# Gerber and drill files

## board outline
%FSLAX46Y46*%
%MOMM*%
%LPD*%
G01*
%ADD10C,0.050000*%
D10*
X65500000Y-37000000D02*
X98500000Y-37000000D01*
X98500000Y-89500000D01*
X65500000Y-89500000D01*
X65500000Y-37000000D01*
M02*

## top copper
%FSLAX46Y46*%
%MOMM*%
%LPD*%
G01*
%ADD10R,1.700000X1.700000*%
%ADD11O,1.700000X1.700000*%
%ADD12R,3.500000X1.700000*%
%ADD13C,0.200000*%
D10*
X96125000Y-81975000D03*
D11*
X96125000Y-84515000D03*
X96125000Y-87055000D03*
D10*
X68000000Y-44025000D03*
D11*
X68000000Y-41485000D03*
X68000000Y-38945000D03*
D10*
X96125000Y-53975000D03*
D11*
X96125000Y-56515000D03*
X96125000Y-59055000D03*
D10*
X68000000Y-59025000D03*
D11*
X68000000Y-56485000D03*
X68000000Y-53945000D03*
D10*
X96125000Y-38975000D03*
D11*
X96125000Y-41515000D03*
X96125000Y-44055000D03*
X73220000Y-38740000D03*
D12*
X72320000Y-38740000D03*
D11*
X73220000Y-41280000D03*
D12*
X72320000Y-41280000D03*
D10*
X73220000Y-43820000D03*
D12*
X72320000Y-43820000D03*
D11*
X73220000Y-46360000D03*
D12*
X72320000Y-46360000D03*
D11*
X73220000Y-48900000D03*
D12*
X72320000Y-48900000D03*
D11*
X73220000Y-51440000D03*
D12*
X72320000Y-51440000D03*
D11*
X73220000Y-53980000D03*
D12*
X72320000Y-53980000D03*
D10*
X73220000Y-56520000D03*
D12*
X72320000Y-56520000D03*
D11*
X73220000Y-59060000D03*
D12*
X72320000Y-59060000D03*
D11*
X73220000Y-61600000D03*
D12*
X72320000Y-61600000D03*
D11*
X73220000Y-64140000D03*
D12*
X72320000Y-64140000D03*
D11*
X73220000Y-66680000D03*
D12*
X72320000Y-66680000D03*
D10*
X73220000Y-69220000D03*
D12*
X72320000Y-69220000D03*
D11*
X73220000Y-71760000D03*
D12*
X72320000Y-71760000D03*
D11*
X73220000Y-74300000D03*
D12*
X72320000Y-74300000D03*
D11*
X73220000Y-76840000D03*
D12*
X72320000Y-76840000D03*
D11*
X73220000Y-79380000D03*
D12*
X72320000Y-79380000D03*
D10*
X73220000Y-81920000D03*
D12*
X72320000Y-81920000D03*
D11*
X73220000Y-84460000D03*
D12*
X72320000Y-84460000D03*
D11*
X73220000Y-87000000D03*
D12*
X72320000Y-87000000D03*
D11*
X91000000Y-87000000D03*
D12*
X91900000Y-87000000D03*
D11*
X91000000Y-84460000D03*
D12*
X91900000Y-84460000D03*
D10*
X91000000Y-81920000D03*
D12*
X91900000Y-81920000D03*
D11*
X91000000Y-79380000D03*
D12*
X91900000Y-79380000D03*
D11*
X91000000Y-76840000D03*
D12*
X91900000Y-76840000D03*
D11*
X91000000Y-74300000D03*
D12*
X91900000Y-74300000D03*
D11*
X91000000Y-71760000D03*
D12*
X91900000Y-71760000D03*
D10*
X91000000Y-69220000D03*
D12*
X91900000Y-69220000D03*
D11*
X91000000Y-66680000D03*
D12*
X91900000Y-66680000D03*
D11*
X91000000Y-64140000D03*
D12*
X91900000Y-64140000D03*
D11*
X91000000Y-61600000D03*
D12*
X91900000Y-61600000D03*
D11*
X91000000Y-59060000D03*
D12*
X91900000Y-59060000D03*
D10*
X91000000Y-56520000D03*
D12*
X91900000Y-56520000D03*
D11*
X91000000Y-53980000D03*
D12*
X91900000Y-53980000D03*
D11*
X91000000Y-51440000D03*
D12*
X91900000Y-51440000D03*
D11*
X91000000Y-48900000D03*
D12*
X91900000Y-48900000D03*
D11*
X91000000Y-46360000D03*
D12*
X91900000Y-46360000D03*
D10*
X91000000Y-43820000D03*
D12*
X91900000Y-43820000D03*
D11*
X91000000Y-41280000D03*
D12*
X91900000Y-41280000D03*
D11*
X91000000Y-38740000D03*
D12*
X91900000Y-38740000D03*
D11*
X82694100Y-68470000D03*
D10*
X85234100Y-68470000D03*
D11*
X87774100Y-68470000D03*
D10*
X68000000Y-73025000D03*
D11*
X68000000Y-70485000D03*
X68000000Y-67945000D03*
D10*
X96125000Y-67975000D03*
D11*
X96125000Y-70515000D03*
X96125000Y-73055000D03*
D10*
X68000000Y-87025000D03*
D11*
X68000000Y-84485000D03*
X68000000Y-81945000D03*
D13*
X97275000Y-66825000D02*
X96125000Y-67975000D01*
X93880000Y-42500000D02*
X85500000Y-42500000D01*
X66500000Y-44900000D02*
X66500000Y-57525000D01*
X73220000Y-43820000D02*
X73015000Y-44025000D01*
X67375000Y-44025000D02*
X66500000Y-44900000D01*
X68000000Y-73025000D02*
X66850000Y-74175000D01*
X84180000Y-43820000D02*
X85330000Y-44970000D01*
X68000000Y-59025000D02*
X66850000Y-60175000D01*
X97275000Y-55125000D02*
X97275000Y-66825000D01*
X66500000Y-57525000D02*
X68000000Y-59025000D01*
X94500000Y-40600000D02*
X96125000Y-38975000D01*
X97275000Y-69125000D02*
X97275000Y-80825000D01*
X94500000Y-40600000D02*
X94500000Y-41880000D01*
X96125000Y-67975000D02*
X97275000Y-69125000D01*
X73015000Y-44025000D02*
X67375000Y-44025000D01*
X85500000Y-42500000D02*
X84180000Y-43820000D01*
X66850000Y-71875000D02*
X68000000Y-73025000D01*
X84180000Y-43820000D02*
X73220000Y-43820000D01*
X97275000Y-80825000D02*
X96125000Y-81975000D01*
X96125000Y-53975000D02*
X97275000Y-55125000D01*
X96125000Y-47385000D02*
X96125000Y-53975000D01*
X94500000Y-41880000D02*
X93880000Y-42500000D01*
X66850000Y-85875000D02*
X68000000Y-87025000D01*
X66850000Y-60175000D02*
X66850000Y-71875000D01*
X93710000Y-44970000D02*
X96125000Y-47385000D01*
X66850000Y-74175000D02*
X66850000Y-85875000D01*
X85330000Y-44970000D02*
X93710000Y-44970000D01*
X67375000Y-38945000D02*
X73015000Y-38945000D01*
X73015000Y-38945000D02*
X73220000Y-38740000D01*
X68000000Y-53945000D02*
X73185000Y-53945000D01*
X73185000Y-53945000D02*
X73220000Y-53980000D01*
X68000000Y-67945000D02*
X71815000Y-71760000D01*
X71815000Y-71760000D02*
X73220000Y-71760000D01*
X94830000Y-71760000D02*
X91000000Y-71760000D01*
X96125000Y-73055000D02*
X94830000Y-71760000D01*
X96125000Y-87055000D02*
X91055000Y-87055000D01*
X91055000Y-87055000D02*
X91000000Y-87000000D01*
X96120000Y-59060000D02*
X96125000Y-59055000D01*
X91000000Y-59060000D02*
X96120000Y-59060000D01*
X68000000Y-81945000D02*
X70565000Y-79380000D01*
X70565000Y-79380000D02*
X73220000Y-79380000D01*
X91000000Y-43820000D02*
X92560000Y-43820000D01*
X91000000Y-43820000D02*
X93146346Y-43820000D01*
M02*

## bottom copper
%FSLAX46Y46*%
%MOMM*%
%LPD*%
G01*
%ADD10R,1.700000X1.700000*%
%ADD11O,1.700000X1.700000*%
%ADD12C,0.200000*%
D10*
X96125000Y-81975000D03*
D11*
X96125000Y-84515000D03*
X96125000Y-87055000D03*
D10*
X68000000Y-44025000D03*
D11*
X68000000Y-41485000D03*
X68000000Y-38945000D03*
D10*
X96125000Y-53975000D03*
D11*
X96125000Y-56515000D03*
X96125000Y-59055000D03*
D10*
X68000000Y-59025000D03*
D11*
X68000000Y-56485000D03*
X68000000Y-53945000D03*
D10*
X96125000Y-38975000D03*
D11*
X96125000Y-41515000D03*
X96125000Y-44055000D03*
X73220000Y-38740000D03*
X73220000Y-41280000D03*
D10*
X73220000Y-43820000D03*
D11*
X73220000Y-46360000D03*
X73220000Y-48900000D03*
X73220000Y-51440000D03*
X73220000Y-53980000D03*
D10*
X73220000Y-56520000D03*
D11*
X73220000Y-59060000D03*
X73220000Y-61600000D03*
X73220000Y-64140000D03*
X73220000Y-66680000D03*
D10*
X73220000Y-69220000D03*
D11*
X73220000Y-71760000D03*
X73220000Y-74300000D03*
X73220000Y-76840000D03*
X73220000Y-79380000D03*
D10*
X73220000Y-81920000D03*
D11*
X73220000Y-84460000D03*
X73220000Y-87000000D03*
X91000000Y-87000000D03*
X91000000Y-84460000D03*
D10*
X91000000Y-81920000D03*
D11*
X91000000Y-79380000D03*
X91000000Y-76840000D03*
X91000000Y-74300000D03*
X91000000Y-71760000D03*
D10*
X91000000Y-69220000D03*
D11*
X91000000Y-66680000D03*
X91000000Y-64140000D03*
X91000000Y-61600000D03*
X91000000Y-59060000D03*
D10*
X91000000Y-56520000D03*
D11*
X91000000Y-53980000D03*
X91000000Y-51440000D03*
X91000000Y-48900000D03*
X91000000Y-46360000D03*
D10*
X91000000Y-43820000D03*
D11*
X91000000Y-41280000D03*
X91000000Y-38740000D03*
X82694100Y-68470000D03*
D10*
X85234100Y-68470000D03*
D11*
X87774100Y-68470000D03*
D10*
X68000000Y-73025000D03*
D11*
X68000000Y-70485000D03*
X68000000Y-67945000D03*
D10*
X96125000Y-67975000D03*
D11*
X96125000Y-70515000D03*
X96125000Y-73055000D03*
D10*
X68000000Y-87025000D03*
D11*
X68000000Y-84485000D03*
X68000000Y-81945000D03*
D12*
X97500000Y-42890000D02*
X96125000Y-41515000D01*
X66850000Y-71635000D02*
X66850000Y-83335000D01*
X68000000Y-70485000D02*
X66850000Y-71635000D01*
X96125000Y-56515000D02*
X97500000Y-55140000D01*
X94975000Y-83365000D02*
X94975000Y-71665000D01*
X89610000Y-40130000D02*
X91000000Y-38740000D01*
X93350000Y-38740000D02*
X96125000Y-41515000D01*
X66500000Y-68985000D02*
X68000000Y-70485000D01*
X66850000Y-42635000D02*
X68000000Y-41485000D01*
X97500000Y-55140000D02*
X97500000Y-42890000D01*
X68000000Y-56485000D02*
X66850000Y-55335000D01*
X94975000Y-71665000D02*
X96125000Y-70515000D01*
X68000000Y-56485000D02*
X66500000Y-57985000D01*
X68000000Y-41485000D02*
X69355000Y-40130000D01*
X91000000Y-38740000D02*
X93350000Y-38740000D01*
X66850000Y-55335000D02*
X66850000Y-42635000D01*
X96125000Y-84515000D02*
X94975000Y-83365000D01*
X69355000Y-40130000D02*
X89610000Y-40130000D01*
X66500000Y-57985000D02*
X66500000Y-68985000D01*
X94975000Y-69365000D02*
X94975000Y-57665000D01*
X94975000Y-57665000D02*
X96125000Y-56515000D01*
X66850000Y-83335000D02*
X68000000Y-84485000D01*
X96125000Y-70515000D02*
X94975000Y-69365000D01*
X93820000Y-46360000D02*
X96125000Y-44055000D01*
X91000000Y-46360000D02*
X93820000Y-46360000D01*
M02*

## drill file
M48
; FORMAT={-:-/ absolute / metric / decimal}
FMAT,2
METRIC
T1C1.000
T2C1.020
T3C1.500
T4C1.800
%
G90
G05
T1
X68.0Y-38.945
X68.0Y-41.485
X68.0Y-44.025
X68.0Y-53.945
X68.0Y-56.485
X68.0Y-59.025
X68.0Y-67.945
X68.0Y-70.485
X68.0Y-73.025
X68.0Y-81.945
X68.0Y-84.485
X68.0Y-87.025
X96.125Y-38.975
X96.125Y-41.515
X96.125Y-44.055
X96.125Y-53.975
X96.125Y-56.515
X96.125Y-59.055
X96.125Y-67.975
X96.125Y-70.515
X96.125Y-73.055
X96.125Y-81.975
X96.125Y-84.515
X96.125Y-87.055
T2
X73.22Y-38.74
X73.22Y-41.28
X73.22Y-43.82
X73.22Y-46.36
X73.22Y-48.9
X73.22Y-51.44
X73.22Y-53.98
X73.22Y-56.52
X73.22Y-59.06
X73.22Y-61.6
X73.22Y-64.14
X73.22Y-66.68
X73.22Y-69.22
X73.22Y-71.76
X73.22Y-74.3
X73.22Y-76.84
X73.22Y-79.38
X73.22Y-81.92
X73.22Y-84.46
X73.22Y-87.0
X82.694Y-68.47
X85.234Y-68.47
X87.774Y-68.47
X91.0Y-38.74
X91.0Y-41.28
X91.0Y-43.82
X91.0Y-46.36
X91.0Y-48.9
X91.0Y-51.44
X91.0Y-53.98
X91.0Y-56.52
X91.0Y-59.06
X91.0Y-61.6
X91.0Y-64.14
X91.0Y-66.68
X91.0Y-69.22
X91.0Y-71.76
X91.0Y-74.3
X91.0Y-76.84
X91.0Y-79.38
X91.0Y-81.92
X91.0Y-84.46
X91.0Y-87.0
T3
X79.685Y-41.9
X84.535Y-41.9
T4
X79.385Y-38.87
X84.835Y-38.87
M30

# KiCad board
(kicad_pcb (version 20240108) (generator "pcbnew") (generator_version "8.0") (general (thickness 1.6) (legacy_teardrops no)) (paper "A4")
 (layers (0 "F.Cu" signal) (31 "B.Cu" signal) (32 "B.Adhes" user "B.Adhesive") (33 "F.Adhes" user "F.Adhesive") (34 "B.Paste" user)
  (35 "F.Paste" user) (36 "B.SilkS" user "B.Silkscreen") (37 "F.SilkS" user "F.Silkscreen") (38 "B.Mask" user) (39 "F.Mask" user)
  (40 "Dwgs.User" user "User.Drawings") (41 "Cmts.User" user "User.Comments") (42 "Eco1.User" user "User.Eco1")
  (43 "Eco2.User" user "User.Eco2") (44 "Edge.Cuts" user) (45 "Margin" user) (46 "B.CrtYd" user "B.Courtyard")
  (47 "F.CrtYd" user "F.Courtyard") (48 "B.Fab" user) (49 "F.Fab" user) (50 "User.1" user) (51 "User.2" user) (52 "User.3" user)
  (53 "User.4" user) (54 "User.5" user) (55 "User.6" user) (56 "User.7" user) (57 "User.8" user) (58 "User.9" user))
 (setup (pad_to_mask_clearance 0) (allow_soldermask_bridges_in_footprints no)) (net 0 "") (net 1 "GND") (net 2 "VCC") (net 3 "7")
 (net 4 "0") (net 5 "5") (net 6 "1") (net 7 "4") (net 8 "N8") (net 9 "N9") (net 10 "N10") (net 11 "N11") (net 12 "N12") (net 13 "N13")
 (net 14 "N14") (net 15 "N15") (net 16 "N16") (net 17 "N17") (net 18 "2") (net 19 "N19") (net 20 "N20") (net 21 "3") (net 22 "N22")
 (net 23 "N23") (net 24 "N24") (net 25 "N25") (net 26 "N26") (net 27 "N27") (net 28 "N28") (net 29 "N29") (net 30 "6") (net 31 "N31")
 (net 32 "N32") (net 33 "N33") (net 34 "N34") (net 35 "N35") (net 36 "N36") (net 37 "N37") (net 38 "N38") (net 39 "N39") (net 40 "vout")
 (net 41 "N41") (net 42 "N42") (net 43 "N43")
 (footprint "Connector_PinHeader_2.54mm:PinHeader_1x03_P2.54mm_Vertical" (layer "F.Cu") (at 96.125 81.975)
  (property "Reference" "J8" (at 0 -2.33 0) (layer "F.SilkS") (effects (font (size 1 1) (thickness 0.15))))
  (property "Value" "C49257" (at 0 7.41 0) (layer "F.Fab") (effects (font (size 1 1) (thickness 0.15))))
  (pad "1" thru_hole rect (at 0 0) (size 1.7 1.7) (drill 1) (layers "*.Cu" "*.Mask") (remove_unused_layers no) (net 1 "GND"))
  (pad "2" thru_hole oval (at 0 2.54) (size 1.7 1.7) (drill 1) (layers "*.Cu" "*.Mask") (remove_unused_layers no) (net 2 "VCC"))
  (pad "3" thru_hole oval (at 0 5.08) (size 1.7 1.7) (drill 1) (layers "*.Cu" "*.Mask") (remove_unused_layers no) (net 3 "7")))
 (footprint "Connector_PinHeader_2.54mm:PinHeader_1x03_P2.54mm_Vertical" (layer "F.Cu") (at 68 44.025 180)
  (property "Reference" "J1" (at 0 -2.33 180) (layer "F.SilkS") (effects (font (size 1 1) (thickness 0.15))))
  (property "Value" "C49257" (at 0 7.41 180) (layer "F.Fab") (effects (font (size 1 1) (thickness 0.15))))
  (pad "1" thru_hole rect (at 0 0 180) (size 1.7 1.7) (drill 1) (layers "*.Cu" "*.Mask") (remove_unused_layers no) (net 1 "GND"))
  (pad "2" thru_hole oval (at 0 2.54 180) (size 1.7 1.7) (drill 1) (layers "*.Cu" "*.Mask") (remove_unused_layers no) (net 2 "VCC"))
  (pad "3" thru_hole oval (at 0 5.08 180) (size 1.7 1.7) (drill 1) (layers "*.Cu" "*.Mask") (remove_unused_layers no) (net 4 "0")))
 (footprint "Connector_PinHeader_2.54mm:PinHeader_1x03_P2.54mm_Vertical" (layer "F.Cu") (at 96.125 53.975)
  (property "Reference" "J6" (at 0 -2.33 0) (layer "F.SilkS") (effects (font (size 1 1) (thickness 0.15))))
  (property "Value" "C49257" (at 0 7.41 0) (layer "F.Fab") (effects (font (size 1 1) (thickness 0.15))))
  (pad "1" thru_hole rect (at 0 0) (size 1.7 1.7) (drill 1) (layers "*.Cu" "*.Mask") (remove_unused_layers no) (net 1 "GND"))
  (pad "2" thru_hole oval (at 0 2.54) (size 1.7 1.7) (drill 1) (layers "*.Cu" "*.Mask") (remove_unused_layers no) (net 2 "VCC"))
  (pad "3" thru_hole oval (at 0 5.08) (size 1.7 1.7) (drill 1) (layers "*.Cu" "*.Mask") (remove_unused_layers no) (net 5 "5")))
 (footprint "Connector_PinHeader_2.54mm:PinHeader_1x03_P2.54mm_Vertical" (layer "F.Cu") (at 68 59.025 180)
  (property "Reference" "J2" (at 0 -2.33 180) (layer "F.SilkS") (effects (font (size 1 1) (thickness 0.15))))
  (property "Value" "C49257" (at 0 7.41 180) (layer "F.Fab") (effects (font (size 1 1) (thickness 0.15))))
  (pad "1" thru_hole rect (at 0 0 180) (size 1.7 1.7) (drill 1) (layers "*.Cu" "*.Mask") (remove_unused_layers no) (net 1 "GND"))
  (pad "2" thru_hole oval (at 0 2.54 180) (size 1.7 1.7) (drill 1) (layers "*.Cu" "*.Mask") (remove_unused_layers no) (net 2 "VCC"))
  (pad "3" thru_hole oval (at 0 5.08 180) (size 1.7 1.7) (drill 1) (layers "*.Cu" "*.Mask") (remove_unused_layers no) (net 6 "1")))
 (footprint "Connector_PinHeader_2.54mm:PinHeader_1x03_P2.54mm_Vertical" (layer "F.Cu") (at 96.125 38.975)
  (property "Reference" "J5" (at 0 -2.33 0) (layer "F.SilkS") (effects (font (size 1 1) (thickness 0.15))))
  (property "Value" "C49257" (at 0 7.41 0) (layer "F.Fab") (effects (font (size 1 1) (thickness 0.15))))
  (pad "1" thru_hole rect (at 0 0) (size 1.7 1.7) (drill 1) (layers "*.Cu" "*.Mask") (remove_unused_layers no) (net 1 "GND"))
  (pad "2" thru_hole oval (at 0 2.54) (size 1.7 1.7) (drill 1) (layers "*.Cu" "*.Mask") (remove_unused_layers no) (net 2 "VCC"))
  (pad "3" thru_hole oval (at 0 5.08) (size 1.7 1.7) (drill 1) (layers "*.Cu" "*.Mask") (remove_unused_layers no) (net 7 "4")))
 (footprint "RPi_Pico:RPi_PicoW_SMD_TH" (layer "F.Cu") (at 82.11 62.87)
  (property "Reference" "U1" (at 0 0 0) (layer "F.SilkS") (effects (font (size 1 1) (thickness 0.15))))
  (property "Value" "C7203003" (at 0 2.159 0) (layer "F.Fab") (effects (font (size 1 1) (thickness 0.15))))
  (pad "" np_thru_hole oval (at -2.725 -24) (size 1.8 1.8) (drill 1.8) (layers "*.Cu" "*.Mask"))
  (pad "" np_thru_hole oval (at -2.425 -20.97) (size 1.5 1.5) (drill 1.5) (layers "*.Cu" "*.Mask"))
  (pad "" np_thru_hole oval (at 2.425 -20.97) (size 1.5 1.5) (drill 1.5) (layers "*.Cu" "*.Mask"))
  (pad "" np_thru_hole oval (at 2.725 -24) (size 1.8 1.8) (drill 1.8) (layers "*.Cu" "*.Mask"))
  (pad "1" thru_hole oval (at -8.89 -24.13) (size 1.7 1.7) (drill 1.02) (layers "*.Cu" "*.Mask") (remove_unused_layers no) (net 4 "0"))
  (pad "1" smd rect (at -8.89 -24.13) (size 3.5 1.7) (drill (offset -0.9 0)) (layers "F.Cu" "F.Mask") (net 4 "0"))
  (pad "2" thru_hole oval (at -8.89 -21.59) (size 1.7 1.7) (drill 1.02) (layers "*.Cu" "*.Mask") (remove_unused_layers no) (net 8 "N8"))
  (pad "2" smd rect (at -8.89 -21.59) (size 3.5 1.7) (drill (offset -0.9 0)) (layers "F.Cu" "F.Mask") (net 8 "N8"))
  (pad "3" thru_hole rect (at -8.89 -19.05) (size 1.7 1.7) (drill 1.02) (layers "*.Cu" "*.Mask") (remove_unused_layers no) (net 1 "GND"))
  (pad "3" smd rect (at -8.89 -19.05) (size 3.5 1.7) (drill (offset -0.9 0)) (layers "F.Cu" "F.Mask") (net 1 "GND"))
  (pad "4" thru_hole oval (at -8.89 -16.51) (size 1.7 1.7) (drill 1.02) (layers "*.Cu" "*.Mask") (remove_unused_layers no) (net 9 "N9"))
  (pad "4" smd rect (at -8.89 -16.51) (size 3.5 1.7) (drill (offset -0.9 0)) (layers "F.Cu" "F.Mask") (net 9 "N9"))
  (pad "5" thru_hole oval (at -8.89 -13.97) (size 1.7 1.7) (drill 1.02) (layers "*.Cu" "*.Mask") (remove_unused_layers no) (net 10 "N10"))
  (pad "5" smd rect (at -8.89 -13.97) (size 3.5 1.7) (drill (offset -0.9 0)) (layers "F.Cu" "F.Mask") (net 10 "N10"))
  (pad "6" thru_hole oval (at -8.89 -11.43) (size 1.7 1.7) (drill 1.02) (layers "*.Cu" "*.Mask") (remove_unused_layers no) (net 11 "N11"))
  (pad "6" smd rect (at -8.89 -11.43) (size 3.5 1.7) (drill (offset -0.9 0)) (layers "F.Cu" "F.Mask") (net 11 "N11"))
  (pad "7" thru_hole oval (at -8.89 -8.89) (size 1.7 1.7) (drill 1.02) (layers "*.Cu" "*.Mask") (remove_unused_layers no) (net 6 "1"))
  (pad "7" smd rect (at -8.89 -8.89) (size 3.5 1.7) (drill (offset -0.9 0)) (layers "F.Cu" "F.Mask") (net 6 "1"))
  (pad "8" thru_hole rect (at -8.89 -6.35) (size 1.7 1.7) (drill 1.02) (layers "*.Cu" "*.Mask") (remove_unused_layers no) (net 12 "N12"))
  (pad "8" smd rect (at -8.89 -6.35) (size 3.5 1.7) (drill (offset -0.9 0)) (layers "F.Cu" "F.Mask") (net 12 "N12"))
  (pad "9" thru_hole oval (at -8.89 -3.81) (size 1.7 1.7) (drill 1.02) (layers "*.Cu" "*.Mask") (remove_unused_layers no) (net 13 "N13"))
  (pad "9" smd rect (at -8.89 -3.81) (size 3.5 1.7) (drill (offset -0.9 0)) (layers "F.Cu" "F.Mask") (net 13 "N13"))
  (pad "10" thru_hole oval (at -8.89 -1.27) (size 1.7 1.7) (drill 1.02) (layers "*.Cu" "*.Mask") (remove_unused_layers no) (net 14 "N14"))
  (pad "10" smd rect (at -8.89 -1.27) (size 3.5 1.7) (drill (offset -0.9 0)) (layers "F.Cu" "F.Mask") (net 14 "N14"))
  (pad "11" thru_hole oval (at -8.89 1.27) (size 1.7 1.7) (drill 1.02) (layers "*.Cu" "*.Mask") (remove_unused_layers no) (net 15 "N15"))
  (pad "11" smd rect (at -8.89 1.27) (size 3.5 1.7) (drill (offset -0.9 0)) (layers "F.Cu" "F.Mask") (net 15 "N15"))
  (pad "12" thru_hole oval (at -8.89 3.81) (size 1.7 1.7) (drill 1.02) (layers "*.Cu" "*.Mask") (remove_unused_layers no) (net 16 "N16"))
  (pad "12" smd rect (at -8.89 3.81) (size 3.5 1.7) (drill (offset -0.9 0)) (layers "F.Cu" "F.Mask") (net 16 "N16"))
  (pad "13" thru_hole rect (at -8.89 6.35) (size 1.7 1.7) (drill 1.02) (layers "*.Cu" "*.Mask") (remove_unused_layers no) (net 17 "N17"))
  (pad "13" smd rect (at -8.89 6.35) (size 3.5 1.7) (drill (offset -0.9 0)) (layers "F.Cu" "F.Mask") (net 17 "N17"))
  (pad "14" thru_hole oval (at -8.89 8.89) (size 1.7 1.7) (drill 1.02) (layers "*.Cu" "*.Mask") (remove_unused_layers no) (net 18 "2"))
  (pad "14" smd rect (at -8.89 8.89) (size 3.5 1.7) (drill (offset -0.9 0)) (layers "F.Cu" "F.Mask") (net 18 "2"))
  (pad "15" thru_hole oval (at -8.89 11.43) (size 1.7 1.7) (drill 1.02) (layers "*.Cu" "*.Mask") (remove_unused_layers no) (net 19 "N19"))
  (pad "15" smd rect (at -8.89 11.43) (size 3.5 1.7) (drill (offset -0.9 0)) (layers "F.Cu" "F.Mask") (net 19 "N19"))
  (pad "16" thru_hole oval (at -8.89 13.97) (size 1.7 1.7) (drill 1.02) (layers "*.Cu" "*.Mask") (remove_unused_layers no) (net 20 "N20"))
  (pad "16" smd rect (at -8.89 13.97) (size 3.5 1.7) (drill (offset -0.9 0)) (layers "F.Cu" "F.Mask") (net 20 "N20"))
  (pad "17" thru_hole oval (at -8.89 16.51) (size 1.7 1.7) (drill 1.02) (layers "*.Cu" "*.Mask") (remove_unused_layers no) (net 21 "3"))
  (pad "17" smd rect (at -8.89 16.51) (size 3.5 1.7) (drill (offset -0.9 0)) (layers "F.Cu" "F.Mask") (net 21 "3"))
  (pad "18" thru_hole rect (at -8.89 19.05) (size 1.7 1.7) (drill 1.02) (layers "*.Cu" "*.Mask") (remove_unused_layers no) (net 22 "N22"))
  (pad "18" smd rect (at -8.89 19.05) (size 3.5 1.7) (drill (offset -0.9 0)) (layers "F.Cu" "F.Mask") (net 22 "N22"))
  (pad "19" thru_hole oval (at -8.89 21.59) (size 1.7 1.7) (drill 1.02) (layers "*.Cu" "*.Mask") (remove_unused_layers no) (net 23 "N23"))
  (pad "19" smd rect (at -8.89 21.59) (size 3.5 1.7) (drill (offset -0.9 0)) (layers "F.Cu" "F.Mask") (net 23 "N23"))
  (pad "20" thru_hole oval (at -8.89 24.13) (size 1.7 1.7) (drill 1.02) (layers "*.Cu" "*.Mask") (remove_unused_layers no) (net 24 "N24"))
  (pad "20" smd rect (at -8.89 24.13) (size 3.5 1.7) (drill (offset -0.9 0)) (layers "F.Cu" "F.Mask") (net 24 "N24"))
  (pad "21" thru_hole oval (at 8.89 24.13) (size 1.7 1.7) (drill 1.02) (layers "*.Cu" "*.Mask") (remove_unused_layers no) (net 3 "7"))
  (pad "21" smd rect (at 8.89 24.13) (size 3.5 1.7) (drill (offset 0.9 0)) (layers "F.Cu" "F.Mask") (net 3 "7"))
  (pad "22" thru_hole oval (at 8.89 21.59) (size 1.7 1.7) (drill 1.02) (layers "*.Cu" "*.Mask") (remove_unused_layers no) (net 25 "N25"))
  (pad "22" smd rect (at 8.89 21.59) (size 3.5 1.7) (drill (offset 0.9 0)) (layers "F.Cu" "F.Mask") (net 25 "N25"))
  (pad "23" thru_hole rect (at 8.89 19.05) (size 1.7 1.7) (drill 1.02) (layers "*.Cu" "*.Mask") (remove_unused_layers no) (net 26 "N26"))
  (pad "23" smd rect (at 8.89 19.05) (size 3.5 1.7) (drill (offset 0.9 0)) (layers "F.Cu" "F.Mask") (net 26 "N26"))
  (pad "24" thru_hole oval (at 8.89 16.51) (size 1.7 1.7) (drill 1.02) (layers "*.Cu" "*.Mask") (remove_unused_layers no) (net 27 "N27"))
  (pad "24" smd rect (at 8.89 16.51) (size 3.5 1.7) (drill (offset 0.9 0)) (layers "F.Cu" "F.Mask") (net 27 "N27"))
  (pad "25" thru_hole oval (at 8.89 13.97) (size 1.7 1.7) (drill 1.02) (layers "*.Cu" "*.Mask") (remove_unused_layers no) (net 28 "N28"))
  (pad "25" smd rect (at 8.89 13.97) (size 3.5 1.7) (drill (offset 0.9 0)) (layers "F.Cu" "F.Mask") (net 28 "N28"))
  (pad "26" thru_hole oval (at 8.89 11.43) (size 1.7 1.7) (drill 1.02) (layers "*.Cu" "*.Mask") (remove_unused_layers no) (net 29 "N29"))
  (pad "26" smd rect (at 8.89 11.43) (size 3.5 1.7) (drill (offset 0.9 0)) (layers "F.Cu" "F.Mask") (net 29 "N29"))
  (pad "27" thru_hole oval (at 8.89 8.89) (size 1.7 1.7) (drill 1.02) (layers "*.Cu" "*.Mask") (remove_unused_layers no) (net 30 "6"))
  (pad "27" smd rect (at 8.89 8.89) (size 3.5 1.7) (drill (offset 0.9 0)) (layers "F.Cu" "F.Mask") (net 30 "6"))
  (pad "28" thru_hole rect (at 8.89 6.35) (size 1.7 1.7) (drill 1.02) (layers "*.Cu" "*.Mask") (remove_unused_layers no) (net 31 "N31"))
  (pad "28" smd rect (at 8.89 6.35) (size 3.5 1.7) (drill (offset 0.9 0)) (layers "F.Cu" "F.Mask") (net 31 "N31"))
  (pad "29" thru_hole oval (at 8.89 3.81) (size 1.7 1.7) (drill 1.02) (layers "*.Cu" "*.Mask") (remove_unused_layers no) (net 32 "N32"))
  (pad "29" smd rect (at 8.89 3.81) (size 3.5 1.7) (drill (offset 0.9 0)) (layers "F.Cu" "F.Mask") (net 32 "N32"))
  (pad "30" thru_hole oval (at 8.89 1.27) (size 1.7 1.7) (drill 1.02) (layers "*.Cu" "*.Mask") (remove_unused_layers no) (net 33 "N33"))
  (pad "30" smd rect (at 8.89 1.27) (size 3.5 1.7) (drill (offset 0.9 0)) (layers "F.Cu" "F.Mask") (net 33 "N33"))
  (pad "31" thru_hole oval (at 8.89 -1.27) (size 1.7 1.7) (drill 1.02) (layers "*.Cu" "*.Mask") (remove_unused_layers no) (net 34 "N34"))
  (pad "31" smd rect (at 8.89 -1.27) (size 3.5 1.7) (drill (offset 0.9 0)) (layers "F.Cu" "F.Mask") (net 34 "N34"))
  (pad "32" thru_hole oval (at 8.89 -3.81) (size 1.7 1.7) (drill 1.02) (layers "*.Cu" "*.Mask") (remove_unused_layers no) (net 5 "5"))
  (pad "32" smd rect (at 8.89 -3.81) (size 3.5 1.7) (drill (offset 0.9 0)) (layers "F.Cu" "F.Mask") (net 5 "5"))
  (pad "33" thru_hole rect (at 8.89 -6.35) (size 1.7 1.7) (drill 1.02) (layers "*.Cu" "*.Mask") (remove_unused_layers no) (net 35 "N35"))
  (pad "33" smd rect (at 8.89 -6.35) (size 3.5 1.7) (drill (offset 0.9 0)) (layers "F.Cu" "F.Mask") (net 35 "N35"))
  (pad "34" thru_hole oval (at 8.89 -8.89) (size 1.7 1.7) (drill 1.02) (layers "*.Cu" "*.Mask") (remove_unused_layers no) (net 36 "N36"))
  (pad "34" smd rect (at 8.89 -8.89) (size 3.5 1.7) (drill (offset 0.9 0)) (layers "F.Cu" "F.Mask") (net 36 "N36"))
  (pad "35" thru_hole oval (at 8.89 -11.43) (size 1.7 1.7) (drill 1.02) (layers "*.Cu" "*.Mask") (remove_unused_layers no) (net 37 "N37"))
  (pad "35" smd rect (at 8.89 -11.43) (size 3.5 1.7) (drill (offset 0.9 0)) (layers "F.Cu" "F.Mask") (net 37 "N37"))
  (pad "36" thru_hole oval (at 8.89 -13.97) (size 1.7 1.7) (drill 1.02) (layers "*.Cu" "*.Mask") (remove_unused_layers no) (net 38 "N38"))
  (pad "36" smd rect (at 8.89 -13.97) (size 3.5 1.7) (drill (offset 0.9 0)) (layers "F.Cu" "F.Mask") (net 38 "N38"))
  (pad "37" thru_hole oval (at 8.89 -16.51) (size 1.7 1.7) (drill 1.02) (layers "*.Cu" "*.Mask") (remove_unused_layers no) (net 7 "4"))
  (pad "37" smd rect (at 8.89 -16.51) (size 3.5 1.7) (drill (offset 0.9 0)) (layers "F.Cu" "F.Mask") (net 7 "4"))
  (pad "38" thru_hole rect (at 8.89 -19.05) (size 1.7 1.7) (drill 1.02) (layers "*.Cu" "*.Mask") (remove_unused_layers no) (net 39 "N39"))
  (pad "38" smd rect (at 8.89 -19.05) (size 3.5 1.7) (drill (offset 0.9 0)) (layers "F.Cu" "F.Mask") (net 39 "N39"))
  (pad "39" thru_hole oval (at 8.89 -21.59) (size 1.7 1.7) (drill 1.02) (layers "*.Cu" "*.Mask") (remove_unused_layers no) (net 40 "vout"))
  (pad "39" smd rect (at 8.89 -21.59) (size 3.5 1.7) (drill (offset 0.9 0)) (layers "F.Cu" "F.Mask") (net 40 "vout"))
  (pad "40" thru_hole oval (at 8.89 -24.13) (size 1.7 1.7) (drill 1.02) (layers "*.Cu" "*.Mask") (remove_unused_layers no) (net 2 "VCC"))
  (pad "40" smd rect (at 8.89 -24.13) (size 3.5 1.7) (drill (offset 0.9 0)) (layers "F.Cu" "F.Mask") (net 2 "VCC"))
  (pad "41" thru_hole oval (at 0.5841 5.6) (size 1.7 1.7) (drill 1.02) (layers "*.Cu" "*.Mask") (remove_unused_layers no) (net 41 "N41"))
  (pad "42" thru_hole rect (at 3.1241 5.6) (size 1.7 1.7) (drill 1.02) (layers "*.Cu" "*.Mask") (remove_unused_layers no) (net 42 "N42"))
  (pad "43" thru_hole oval (at 5.6641 5.6) (size 1.7 1.7) (drill 1.02) (layers "*.Cu" "*.Mask") (remove_unused_layers no) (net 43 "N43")))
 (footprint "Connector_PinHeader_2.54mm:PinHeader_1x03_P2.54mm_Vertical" (layer "F.Cu") (at 68 73.025 180)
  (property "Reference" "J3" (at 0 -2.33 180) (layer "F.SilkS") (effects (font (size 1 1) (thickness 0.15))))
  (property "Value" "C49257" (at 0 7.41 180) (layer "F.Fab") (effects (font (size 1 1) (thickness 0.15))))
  (pad "1" thru_hole rect (at 0 0 180) (size 1.7 1.7) (drill 1) (layers "*.Cu" "*.Mask") (remove_unused_layers no) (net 1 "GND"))
  (pad "2" thru_hole oval (at 0 2.54 180) (size 1.7 1.7) (drill 1) (layers "*.Cu" "*.Mask") (remove_unused_layers no) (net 2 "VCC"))
  (pad "3" thru_hole oval (at 0 5.08 180) (size 1.7 1.7) (drill 1) (layers "*.Cu" "*.Mask") (remove_unused_layers no) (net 18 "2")))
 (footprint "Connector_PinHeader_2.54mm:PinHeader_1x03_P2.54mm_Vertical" (layer "F.Cu") (at 96.125 67.975)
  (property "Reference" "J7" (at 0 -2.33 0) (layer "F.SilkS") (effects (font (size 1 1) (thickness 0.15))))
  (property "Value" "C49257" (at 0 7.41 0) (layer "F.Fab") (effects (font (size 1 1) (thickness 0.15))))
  (pad "1" thru_hole rect (at 0 0) (size 1.7 1.7) (drill 1) (layers "*.Cu" "*.Mask") (remove_unused_layers no) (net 1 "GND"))
  (pad "2" thru_hole oval (at 0 2.54) (size 1.7 1.7) (drill 1) (layers "*.Cu" "*.Mask") (remove_unused_layers no) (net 2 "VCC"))
  (pad "3" thru_hole oval (at 0 5.08) (size 1.7 1.7) (drill 1) (layers "*.Cu" "*.Mask") (remove_unused_layers no) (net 30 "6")))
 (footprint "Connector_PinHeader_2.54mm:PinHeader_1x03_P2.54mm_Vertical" (layer "F.Cu") (at 68 87.025 180)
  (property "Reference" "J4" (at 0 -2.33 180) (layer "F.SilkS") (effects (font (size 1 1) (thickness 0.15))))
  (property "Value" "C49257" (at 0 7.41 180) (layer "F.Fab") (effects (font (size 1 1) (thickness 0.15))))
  (pad "1" thru_hole rect (at 0 0 180) (size 1.7 1.7) (drill 1) (layers "*.Cu" "*.Mask") (remove_unused_layers no) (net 1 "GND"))
  (pad "2" thru_hole oval (at 0 2.54 180) (size 1.7 1.7) (drill 1) (layers "*.Cu" "*.Mask") (remove_unused_layers no) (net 2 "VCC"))
  (pad "3" thru_hole oval (at 0 5.08 180) (size 1.7 1.7) (drill 1) (layers "*.Cu" "*.Mask") (remove_unused_layers no) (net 21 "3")))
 (gr_rect (start 65.5 37) (end 98.5 89.5) (stroke (width 0.05) (type default)) (fill none) (layer "Edge.Cuts"))
 (segment (start 97.275 66.825) (end 96.125 67.975) (width 0.2) (layer "F.Cu") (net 1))
 (segment (start 93.88 42.5) (end 85.5 42.5) (width 0.2) (layer "F.Cu") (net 1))
 (segment (start 66.5 44.9) (end 66.5 57.525) (width 0.2) (layer "F.Cu") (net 1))
 (segment (start 73.22 43.82) (end 73.015 44.025) (width 0.2) (layer "F.Cu") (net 1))
 (segment (start 67.375 44.025) (end 66.5 44.9) (width 0.2) (layer "F.Cu") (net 1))
 (segment (start 68 73.025) (end 66.85 74.175) (width 0.2) (layer "F.Cu") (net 1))
 (segment (start 84.18 43.82) (end 85.33 44.97) (width 0.2) (layer "F.Cu") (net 1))
 (segment (start 68 59.025) (end 66.85 60.175) (width 0.2) (layer "F.Cu") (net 1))
 (segment (start 97.275 55.125) (end 97.275 66.825) (width 0.2) (layer "F.Cu") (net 1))
 (segment (start 66.5 57.525) (end 68 59.025) (width 0.2) (layer "F.Cu") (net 1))
 (segment (start 94.5 40.6) (end 96.125 38.975) (width 0.2) (layer "F.Cu") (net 1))
 (segment (start 97.275 69.125) (end 97.275 80.825) (width 0.2) (layer "F.Cu") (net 1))
 (segment (start 94.5 40.6) (end 94.5 41.88) (width 0.2) (layer "F.Cu") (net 1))
 (segment (start 96.125 67.975) (end 97.275 69.125) (width 0.2) (layer "F.Cu") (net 1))
 (segment (start 73.015 44.025) (end 67.375 44.025) (width 0.2) (layer "F.Cu") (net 1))
 (segment (start 85.5 42.5) (end 84.18 43.82) (width 0.2) (layer "F.Cu") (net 1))
 (segment (start 66.85 71.875) (end 68 73.025) (width 0.2) (layer "F.Cu") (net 1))
 (segment (start 84.18 43.82) (end 73.22 43.82) (width 0.2) (layer "F.Cu") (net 1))
 (segment (start 97.275 80.825) (end 96.125 81.975) (width 0.2) (layer "F.Cu") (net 1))
 (segment (start 96.125 53.975) (end 97.275 55.125) (width 0.2) (layer "F.Cu") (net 1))
 (segment (start 96.125 47.385) (end 96.125 53.975) (width 0.2) (layer "F.Cu") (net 1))
 (segment (start 94.5 41.88) (end 93.88 42.5) (width 0.2) (layer "F.Cu") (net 1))
 (segment (start 66.85 85.875) (end 68 87.025) (width 0.2) (layer "F.Cu") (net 1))
 (segment (start 66.85 60.175) (end 66.85 71.875) (width 0.2) (layer "F.Cu") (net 1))
 (segment (start 93.71 44.97) (end 96.125 47.385) (width 0.2) (layer "F.Cu") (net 1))
 (segment (start 66.85 74.175) (end 66.85 85.875) (width 0.2) (layer "F.Cu") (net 1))
 (segment (start 85.33 44.97) (end 93.71 44.97) (width 0.2) (layer "F.Cu") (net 1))
 (segment (start 67.375 38.945) (end 73.015 38.945) (width 0.2) (layer "F.Cu") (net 4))
 (segment (start 73.015 38.945) (end 73.22 38.74) (width 0.2) (layer "F.Cu") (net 4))
 (segment (start 97.5 42.89) (end 96.125 41.515) (width 0.2) (layer "B.Cu") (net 2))
 (segment (start 66.85 71.635) (end 66.85 83.335) (width 0.2) (layer "B.Cu") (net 2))
 (segment (start 68 70.485) (end 66.85 71.635) (width 0.2) (layer "B.Cu") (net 2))
 (segment (start 96.125 56.515) (end 97.5 55.14) (width 0.2) (layer "B.Cu") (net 2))
 (segment (start 94.975 83.365) (end 94.975 71.665) (width 0.2) (layer "B.Cu") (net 2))
 (segment (start 89.61 40.13) (end 91 38.74) (width 0.2) (layer "B.Cu") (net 2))
 (segment (start 93.35 38.74) (end 96.125 41.515) (width 0.2) (layer "B.Cu") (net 2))
 (segment (start 66.5 68.985) (end 68 70.485) (width 0.2) (layer "B.Cu") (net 2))
 (segment (start 66.85 42.635) (end 68 41.485) (width 0.2) (layer "B.Cu") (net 2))
 (segment (start 97.5 55.14) (end 97.5 42.89) (width 0.2) (layer "B.Cu") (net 2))
 (segment (start 68 56.485) (end 66.85 55.335) (width 0.2) (layer "B.Cu") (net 2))
 (segment (start 94.975 71.665) (end 96.125 70.515) (width 0.2) (layer "B.Cu") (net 2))
 (segment (start 68 56.485) (end 66.5 57.985) (width 0.2) (layer "B.Cu") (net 2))
 (segment (start 68 41.485) (end 69.355 40.13) (width 0.2) (layer "B.Cu") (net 2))
 (segment (start 91 38.74) (end 93.35 38.74) (width 0.2) (layer "B.Cu") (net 2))
 (segment (start 66.85 55.335) (end 66.85 42.635) (width 0.2) (layer "B.Cu") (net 2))
 (segment (start 96.125 84.515) (end 94.975 83.365) (width 0.2) (layer "B.Cu") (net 2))
 (segment (start 69.355 40.13) (end 89.61 40.13) (width 0.2) (layer "B.Cu") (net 2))
 (segment (start 66.5 57.985) (end 66.5 68.985) (width 0.2) (layer "B.Cu") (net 2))
 (segment (start 94.975 69.365) (end 94.975 57.665) (width 0.2) (layer "B.Cu") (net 2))
 (segment (start 94.975 57.665) (end 96.125 56.515) (width 0.2) (layer "B.Cu") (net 2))
 (segment (start 66.85 83.335) (end 68 84.485) (width 0.2) (layer "B.Cu") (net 2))
 (segment (start 96.125 70.515) (end 94.975 69.365) (width 0.2) (layer "B.Cu") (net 2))
 (segment (start 68 53.945) (end 73.185 53.945) (width 0.2) (layer "F.Cu") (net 6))
 (segment (start 73.185 53.945) (end 73.22 53.98) (width 0.2) (layer "F.Cu") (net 6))
 (segment (start 68 67.945) (end 71.815 71.76) (width 0.2) (layer "F.Cu") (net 18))
 (segment (start 71.815 71.76) (end 73.22 71.76) (width 0.2) (layer "F.Cu") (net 18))
 (segment (start 94.83 71.76) (end 91 71.76) (width 0.2) (layer "F.Cu") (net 30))
 (segment (start 96.125 73.055) (end 94.83 71.76) (width 0.2) (layer "F.Cu") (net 30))
 (segment (start 96.125 87.055) (end 91.055 87.055) (width 0.2) (layer "F.Cu") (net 3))
 (segment (start 91.055 87.055) (end 91 87) (width 0.2) (layer "F.Cu") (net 3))
 (segment (start 96.12 59.06) (end 96.125 59.055) (width 0.2) (layer "F.Cu") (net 5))
 (segment (start 91 59.06) (end 96.12 59.06) (width 0.2) (layer "F.Cu") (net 5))
 (segment (start 68 81.945) (end 70.565 79.38) (width 0.2) (layer "F.Cu") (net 21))
 (segment (start 70.565 79.38) (end 73.22 79.38) (width 0.2) (layer "F.Cu") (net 21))
 (segment (start 93.82 46.36) (end 96.125 44.055) (width 0.2) (layer "B.Cu") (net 7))
 (segment (start 91 46.36) (end 93.82 46.36) (width 0.2) (layer "B.Cu") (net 7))
 (segment (start 91 43.82) (end 92.56 43.82) (width 0.2) (layer "F.Cu") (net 39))
 (segment (start 91 43.82) (end 93.146346 43.82) (width 0.2) (layer "F.Cu") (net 39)))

